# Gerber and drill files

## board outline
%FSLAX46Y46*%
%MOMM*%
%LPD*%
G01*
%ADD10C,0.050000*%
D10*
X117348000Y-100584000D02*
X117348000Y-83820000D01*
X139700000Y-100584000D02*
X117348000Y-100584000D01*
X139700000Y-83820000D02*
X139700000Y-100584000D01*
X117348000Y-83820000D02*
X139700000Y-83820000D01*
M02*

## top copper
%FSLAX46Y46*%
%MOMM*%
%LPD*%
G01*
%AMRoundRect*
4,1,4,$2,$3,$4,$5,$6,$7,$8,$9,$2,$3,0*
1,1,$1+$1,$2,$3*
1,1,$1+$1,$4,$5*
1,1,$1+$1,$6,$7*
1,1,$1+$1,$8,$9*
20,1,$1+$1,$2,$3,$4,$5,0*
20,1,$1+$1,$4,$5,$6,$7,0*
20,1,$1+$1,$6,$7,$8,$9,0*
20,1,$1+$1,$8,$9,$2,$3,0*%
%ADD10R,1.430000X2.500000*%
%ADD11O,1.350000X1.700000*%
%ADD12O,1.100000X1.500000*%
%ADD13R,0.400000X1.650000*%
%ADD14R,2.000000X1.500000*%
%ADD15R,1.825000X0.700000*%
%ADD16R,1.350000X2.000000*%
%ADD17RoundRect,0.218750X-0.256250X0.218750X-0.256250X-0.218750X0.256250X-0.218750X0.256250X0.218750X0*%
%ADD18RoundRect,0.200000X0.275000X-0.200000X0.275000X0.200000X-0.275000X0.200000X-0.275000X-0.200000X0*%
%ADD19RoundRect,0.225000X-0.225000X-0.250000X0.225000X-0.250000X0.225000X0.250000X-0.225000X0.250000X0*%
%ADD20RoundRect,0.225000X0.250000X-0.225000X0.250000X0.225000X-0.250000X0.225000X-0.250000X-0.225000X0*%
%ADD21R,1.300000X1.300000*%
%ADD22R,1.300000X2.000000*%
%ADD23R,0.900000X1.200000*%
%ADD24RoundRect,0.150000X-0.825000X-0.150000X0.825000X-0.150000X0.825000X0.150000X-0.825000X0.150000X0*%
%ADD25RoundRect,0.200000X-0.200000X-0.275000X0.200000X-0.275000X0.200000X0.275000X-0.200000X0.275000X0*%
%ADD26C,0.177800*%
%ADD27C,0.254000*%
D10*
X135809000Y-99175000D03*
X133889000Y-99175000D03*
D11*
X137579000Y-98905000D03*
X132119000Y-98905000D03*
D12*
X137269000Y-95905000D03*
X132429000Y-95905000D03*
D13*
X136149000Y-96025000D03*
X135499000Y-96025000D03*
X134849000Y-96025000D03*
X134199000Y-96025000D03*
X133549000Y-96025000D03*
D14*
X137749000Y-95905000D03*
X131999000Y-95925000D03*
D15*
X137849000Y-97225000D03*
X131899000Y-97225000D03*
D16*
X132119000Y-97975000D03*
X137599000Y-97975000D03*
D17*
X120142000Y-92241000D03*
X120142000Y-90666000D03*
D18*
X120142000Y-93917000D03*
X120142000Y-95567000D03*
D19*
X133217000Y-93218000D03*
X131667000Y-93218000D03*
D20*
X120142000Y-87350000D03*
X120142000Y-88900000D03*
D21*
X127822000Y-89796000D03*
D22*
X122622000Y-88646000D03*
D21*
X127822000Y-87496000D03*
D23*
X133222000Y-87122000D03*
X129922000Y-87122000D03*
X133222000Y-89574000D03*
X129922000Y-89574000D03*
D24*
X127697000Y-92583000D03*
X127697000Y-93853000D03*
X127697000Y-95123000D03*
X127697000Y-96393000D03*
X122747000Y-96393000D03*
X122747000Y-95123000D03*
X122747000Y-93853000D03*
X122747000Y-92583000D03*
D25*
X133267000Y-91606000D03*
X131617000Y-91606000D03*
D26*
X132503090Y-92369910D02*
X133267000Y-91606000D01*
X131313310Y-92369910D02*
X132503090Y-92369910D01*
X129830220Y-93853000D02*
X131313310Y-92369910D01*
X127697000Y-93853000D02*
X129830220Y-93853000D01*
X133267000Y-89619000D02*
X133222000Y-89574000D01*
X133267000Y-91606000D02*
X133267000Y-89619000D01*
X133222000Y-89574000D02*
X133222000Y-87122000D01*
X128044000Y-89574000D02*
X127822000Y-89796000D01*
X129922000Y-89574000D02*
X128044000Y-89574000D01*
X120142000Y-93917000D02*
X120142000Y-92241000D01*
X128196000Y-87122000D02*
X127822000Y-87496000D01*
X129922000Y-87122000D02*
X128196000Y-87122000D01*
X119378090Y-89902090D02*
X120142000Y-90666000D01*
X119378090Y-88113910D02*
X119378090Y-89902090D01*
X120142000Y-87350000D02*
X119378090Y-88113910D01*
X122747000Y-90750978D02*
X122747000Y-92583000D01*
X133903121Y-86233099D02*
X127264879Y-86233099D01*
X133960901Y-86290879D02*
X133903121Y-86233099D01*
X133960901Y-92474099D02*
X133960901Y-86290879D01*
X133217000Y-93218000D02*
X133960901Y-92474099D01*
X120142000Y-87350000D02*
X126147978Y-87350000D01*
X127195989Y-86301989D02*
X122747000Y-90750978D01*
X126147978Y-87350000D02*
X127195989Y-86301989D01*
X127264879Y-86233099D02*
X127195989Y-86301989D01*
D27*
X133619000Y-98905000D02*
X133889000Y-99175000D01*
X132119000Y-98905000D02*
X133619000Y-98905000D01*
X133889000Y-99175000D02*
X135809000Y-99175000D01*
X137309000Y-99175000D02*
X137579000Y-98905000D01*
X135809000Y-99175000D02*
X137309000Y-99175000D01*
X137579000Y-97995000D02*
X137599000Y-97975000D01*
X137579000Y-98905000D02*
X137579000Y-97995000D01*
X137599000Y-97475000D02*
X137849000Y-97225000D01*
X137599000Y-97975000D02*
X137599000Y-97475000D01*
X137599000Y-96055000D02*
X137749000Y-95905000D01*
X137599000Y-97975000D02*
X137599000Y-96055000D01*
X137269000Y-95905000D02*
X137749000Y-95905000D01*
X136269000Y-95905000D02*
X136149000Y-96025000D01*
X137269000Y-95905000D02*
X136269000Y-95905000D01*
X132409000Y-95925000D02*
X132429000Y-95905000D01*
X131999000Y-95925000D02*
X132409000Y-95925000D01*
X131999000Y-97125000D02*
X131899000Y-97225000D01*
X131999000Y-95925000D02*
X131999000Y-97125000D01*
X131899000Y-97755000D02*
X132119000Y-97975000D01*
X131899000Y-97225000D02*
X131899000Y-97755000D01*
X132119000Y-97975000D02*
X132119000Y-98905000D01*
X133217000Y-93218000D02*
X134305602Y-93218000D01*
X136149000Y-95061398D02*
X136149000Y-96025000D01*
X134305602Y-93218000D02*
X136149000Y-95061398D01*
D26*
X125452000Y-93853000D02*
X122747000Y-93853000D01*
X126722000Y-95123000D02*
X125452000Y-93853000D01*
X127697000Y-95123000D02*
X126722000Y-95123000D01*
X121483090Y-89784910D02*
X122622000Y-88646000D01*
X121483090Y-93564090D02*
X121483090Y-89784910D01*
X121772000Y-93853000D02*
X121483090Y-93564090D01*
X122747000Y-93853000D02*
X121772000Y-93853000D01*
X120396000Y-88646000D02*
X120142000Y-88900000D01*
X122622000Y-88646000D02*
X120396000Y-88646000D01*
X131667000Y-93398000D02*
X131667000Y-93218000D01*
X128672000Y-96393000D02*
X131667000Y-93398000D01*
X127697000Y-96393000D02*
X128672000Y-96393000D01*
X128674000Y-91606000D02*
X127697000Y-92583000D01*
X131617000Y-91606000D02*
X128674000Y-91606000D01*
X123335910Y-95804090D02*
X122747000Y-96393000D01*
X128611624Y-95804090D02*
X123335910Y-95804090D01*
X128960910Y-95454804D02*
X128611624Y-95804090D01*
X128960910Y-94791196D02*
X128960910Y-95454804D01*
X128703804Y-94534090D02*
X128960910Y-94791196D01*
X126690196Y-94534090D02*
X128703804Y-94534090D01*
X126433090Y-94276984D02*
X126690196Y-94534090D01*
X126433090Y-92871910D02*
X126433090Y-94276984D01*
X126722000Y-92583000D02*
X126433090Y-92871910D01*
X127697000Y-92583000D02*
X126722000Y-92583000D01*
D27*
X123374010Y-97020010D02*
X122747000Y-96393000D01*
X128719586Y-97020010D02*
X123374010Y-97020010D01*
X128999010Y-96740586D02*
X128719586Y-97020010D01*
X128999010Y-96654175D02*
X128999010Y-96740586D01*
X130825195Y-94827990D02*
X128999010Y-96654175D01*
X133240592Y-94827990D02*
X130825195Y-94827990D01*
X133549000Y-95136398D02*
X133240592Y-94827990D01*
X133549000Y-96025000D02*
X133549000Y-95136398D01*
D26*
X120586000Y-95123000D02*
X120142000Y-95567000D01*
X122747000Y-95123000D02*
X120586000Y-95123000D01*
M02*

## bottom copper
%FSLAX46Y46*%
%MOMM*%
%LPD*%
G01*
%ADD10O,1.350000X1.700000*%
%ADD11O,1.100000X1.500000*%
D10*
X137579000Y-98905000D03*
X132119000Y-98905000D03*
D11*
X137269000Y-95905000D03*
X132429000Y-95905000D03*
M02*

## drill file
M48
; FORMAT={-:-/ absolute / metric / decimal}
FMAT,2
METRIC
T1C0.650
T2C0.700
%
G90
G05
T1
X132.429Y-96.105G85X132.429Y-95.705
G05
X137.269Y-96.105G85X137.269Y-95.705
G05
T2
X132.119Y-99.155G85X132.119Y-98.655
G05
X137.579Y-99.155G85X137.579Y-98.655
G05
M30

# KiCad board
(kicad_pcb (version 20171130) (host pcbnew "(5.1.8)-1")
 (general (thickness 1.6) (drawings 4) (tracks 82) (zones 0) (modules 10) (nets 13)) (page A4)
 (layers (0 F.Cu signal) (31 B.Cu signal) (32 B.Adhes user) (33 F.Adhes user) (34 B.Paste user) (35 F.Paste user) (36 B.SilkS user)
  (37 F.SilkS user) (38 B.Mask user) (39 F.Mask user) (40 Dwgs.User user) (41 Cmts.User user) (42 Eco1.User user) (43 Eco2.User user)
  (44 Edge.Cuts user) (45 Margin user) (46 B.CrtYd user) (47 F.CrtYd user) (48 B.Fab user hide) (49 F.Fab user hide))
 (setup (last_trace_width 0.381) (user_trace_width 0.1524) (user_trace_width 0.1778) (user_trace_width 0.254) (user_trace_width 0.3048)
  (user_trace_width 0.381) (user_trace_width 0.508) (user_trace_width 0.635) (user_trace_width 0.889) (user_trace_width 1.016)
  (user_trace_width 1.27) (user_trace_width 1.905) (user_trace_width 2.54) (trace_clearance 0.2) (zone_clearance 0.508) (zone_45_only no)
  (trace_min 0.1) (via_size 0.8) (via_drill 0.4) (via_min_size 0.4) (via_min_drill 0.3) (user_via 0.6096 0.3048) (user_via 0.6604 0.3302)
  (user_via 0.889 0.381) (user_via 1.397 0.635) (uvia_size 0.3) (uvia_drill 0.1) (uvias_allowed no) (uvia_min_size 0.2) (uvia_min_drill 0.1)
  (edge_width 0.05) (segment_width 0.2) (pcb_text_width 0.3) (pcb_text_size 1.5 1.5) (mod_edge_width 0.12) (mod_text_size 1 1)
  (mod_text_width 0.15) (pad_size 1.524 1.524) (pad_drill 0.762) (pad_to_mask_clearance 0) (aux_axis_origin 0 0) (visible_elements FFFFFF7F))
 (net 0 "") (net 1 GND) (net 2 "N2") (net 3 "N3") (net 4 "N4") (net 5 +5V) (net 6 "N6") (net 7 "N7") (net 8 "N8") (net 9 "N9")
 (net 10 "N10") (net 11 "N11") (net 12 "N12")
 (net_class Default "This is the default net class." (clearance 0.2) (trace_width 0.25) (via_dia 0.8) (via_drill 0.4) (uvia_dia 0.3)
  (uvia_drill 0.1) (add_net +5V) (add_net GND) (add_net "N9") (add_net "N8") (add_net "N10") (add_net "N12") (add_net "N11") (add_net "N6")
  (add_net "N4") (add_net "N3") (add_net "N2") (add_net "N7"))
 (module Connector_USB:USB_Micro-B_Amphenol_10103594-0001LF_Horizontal (layer F.Cu) (at 134.874 97.79)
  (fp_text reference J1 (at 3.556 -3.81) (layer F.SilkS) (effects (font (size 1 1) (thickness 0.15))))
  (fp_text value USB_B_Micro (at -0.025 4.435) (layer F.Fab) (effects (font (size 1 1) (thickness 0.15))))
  (pad 6 smd rect (at 0.935 1.385 90) (size 2.5 1.43) (layers F.Cu F.Paste F.Mask) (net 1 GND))
  (pad 6 smd rect (at -0.985 1.385 90) (size 2.5 1.43) (layers F.Cu F.Paste F.Mask) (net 1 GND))
  (pad 6 thru_hole oval (at 2.705 1.115 90) (size 1.7 1.35) (drill oval 1.2 0.7) (layers *.Cu *.Mask) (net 1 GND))
  (pad 6 thru_hole oval (at -2.755 1.115 90) (size 1.7 1.35) (drill oval 1.2 0.7) (layers *.Cu *.Mask) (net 1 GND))
  (pad 6 thru_hole oval (at 2.395 -1.885 90) (size 1.5 1.1) (drill oval 1.05 0.65) (layers *.Cu *.Mask) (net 1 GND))
  (pad 6 thru_hole oval (at -2.445 -1.885 90) (size 1.5 1.1) (drill oval 1.05 0.65) (layers *.Cu *.Mask) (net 1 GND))
  (pad 5 smd rect (at 1.275 -1.765 90) (size 1.65 0.4) (layers F.Cu F.Paste F.Mask) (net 1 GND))
  (pad 4 smd rect (at 0.625 -1.765 90) (size 1.65 0.4) (layers F.Cu F.Paste F.Mask) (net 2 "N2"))
  (pad 3 smd rect (at -0.025 -1.765 90) (size 1.65 0.4) (layers F.Cu F.Paste F.Mask) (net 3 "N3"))
  (pad 2 smd rect (at -0.675 -1.765 90) (size 1.65 0.4) (layers F.Cu F.Paste F.Mask) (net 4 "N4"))
  (pad 1 smd rect (at -1.325 -1.765 90) (size 1.65 0.4) (layers F.Cu F.Paste F.Mask) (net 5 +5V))
  (pad 6 smd rect (at 2.875 -1.885) (size 2 1.5) (layers F.Cu F.Paste F.Mask) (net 1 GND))
  (pad 6 smd rect (at -2.875 -1.865) (size 2 1.5) (layers F.Cu F.Paste F.Mask) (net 1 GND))
  (pad 6 smd rect (at 2.975 -0.565) (size 1.825 0.7) (layers F.Cu F.Paste F.Mask) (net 1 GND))
  (pad 6 smd rect (at -2.975 -0.565) (size 1.825 0.7) (layers F.Cu F.Paste F.Mask) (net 1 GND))
  (pad 6 smd rect (at -2.755 0.185) (size 1.35 2) (layers F.Cu F.Paste F.Mask) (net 1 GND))
  (pad 6 smd rect (at 2.725 0.185) (size 1.35 2) (layers F.Cu F.Paste F.Mask) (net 1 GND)))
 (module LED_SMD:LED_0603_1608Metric (layer F.Cu) (at 120.142 91.4535 270)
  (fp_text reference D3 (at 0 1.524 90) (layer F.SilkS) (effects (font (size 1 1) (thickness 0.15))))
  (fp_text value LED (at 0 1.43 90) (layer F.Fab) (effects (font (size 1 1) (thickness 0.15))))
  (pad 2 smd roundrect (at 0.7875 0 270) (size 0.875 0.95) (layers F.Cu F.Paste F.Mask) (roundrect_rratio 0.25) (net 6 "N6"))
  (pad 1 smd roundrect (at -0.7875 0 270) (size 0.875 0.95) (layers F.Cu F.Paste F.Mask) (roundrect_rratio 0.25) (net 1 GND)))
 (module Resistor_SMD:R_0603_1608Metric (layer F.Cu) (at 120.142 94.742 90)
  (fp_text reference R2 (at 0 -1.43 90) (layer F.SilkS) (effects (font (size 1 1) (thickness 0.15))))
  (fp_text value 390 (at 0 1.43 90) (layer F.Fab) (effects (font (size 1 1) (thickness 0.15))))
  (pad 2 smd roundrect (at 0.825 0 90) (size 0.8 0.95) (layers F.Cu F.Paste F.Mask) (roundrect_rratio 0.25) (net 6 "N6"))
  (pad 1 smd roundrect (at -0.825 0 90) (size 0.8 0.95) (layers F.Cu F.Paste F.Mask) (roundrect_rratio 0.25) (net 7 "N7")))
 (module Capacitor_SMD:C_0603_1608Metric (layer F.Cu) (at 132.442 93.218)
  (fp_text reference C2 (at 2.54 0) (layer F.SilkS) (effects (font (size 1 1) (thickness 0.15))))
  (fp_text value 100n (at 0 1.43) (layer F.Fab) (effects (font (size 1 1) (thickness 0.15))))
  (pad 2 smd roundrect (at 0.775 0) (size 0.9 0.95) (layers F.Cu F.Paste F.Mask) (roundrect_rratio 0.25) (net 1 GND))
  (pad 1 smd roundrect (at -0.775 0) (size 0.9 0.95) (layers F.Cu F.Paste F.Mask) (roundrect_rratio 0.25) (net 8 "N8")))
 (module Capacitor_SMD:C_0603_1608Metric (layer F.Cu) (at 120.142 88.125 90)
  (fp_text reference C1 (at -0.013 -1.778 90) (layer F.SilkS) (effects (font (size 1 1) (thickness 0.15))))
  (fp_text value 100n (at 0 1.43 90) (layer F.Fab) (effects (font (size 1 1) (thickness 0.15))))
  (pad 2 smd roundrect (at 0.775 0 90) (size 0.9 0.95) (layers F.Cu F.Paste F.Mask) (roundrect_rratio 0.25) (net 1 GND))
  (pad 1 smd roundrect (at -0.775 0 90) (size 0.9 0.95) (layers F.Cu F.Paste F.Mask) (roundrect_rratio 0.25) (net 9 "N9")))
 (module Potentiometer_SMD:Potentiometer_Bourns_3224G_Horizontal (layer F.Cu) (at 125.222 88.646)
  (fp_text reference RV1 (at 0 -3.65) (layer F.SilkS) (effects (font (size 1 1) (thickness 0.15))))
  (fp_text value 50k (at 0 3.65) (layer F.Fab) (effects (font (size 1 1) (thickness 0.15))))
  (pad 3 smd rect (at 2.6 1.15) (size 1.3 1.3) (layers F.Cu F.Paste F.Mask) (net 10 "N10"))
  (pad 2 smd rect (at -2.6 0) (size 1.3 2) (layers F.Cu F.Paste F.Mask) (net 9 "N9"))
  (pad 1 smd rect (at 2.6 -1.15) (size 1.3 1.3) (layers F.Cu F.Paste F.Mask) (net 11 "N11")))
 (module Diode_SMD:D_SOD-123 (layer F.Cu) (at 131.572 87.122)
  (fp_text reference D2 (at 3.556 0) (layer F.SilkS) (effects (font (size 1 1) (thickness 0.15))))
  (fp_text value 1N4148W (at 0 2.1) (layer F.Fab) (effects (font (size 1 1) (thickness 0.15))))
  (pad 2 smd rect (at 1.65 0) (size 0.9 1.2) (layers F.Cu F.Paste F.Mask) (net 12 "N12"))
  (pad 1 smd rect (at -1.65 0) (size 0.9 1.2) (layers F.Cu F.Paste F.Mask) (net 11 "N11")))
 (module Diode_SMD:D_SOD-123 (layer F.Cu) (at 131.572 89.574)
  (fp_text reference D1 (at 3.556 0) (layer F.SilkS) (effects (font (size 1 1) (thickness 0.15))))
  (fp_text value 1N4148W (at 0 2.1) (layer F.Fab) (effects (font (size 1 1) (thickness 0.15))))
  (pad 2 smd rect (at 1.65 0) (size 0.9 1.2) (layers F.Cu F.Paste F.Mask) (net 12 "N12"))
  (pad 1 smd rect (at -1.65 0) (size 0.9 1.2) (layers F.Cu F.Paste F.Mask) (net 10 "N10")))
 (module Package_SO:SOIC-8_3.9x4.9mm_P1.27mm (layer F.Cu) (at 125.222 94.488)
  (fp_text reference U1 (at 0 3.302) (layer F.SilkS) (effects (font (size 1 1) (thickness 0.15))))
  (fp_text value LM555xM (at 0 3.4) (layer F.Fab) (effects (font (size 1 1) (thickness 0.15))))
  (pad 8 smd roundrect (at 2.475 -1.905) (size 1.95 0.6) (layers F.Cu F.Paste F.Mask) (roundrect_rratio 0.25) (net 5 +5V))
  (pad 7 smd roundrect (at 2.475 -0.635) (size 1.95 0.6) (layers F.Cu F.Paste F.Mask) (roundrect_rratio 0.25) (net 12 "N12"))
  (pad 6 smd roundrect (at 2.475 0.635) (size 1.95 0.6) (layers F.Cu F.Paste F.Mask) (roundrect_rratio 0.25) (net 9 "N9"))
  (pad 5 smd roundrect (at 2.475 1.905) (size 1.95 0.6) (layers F.Cu F.Paste F.Mask) (roundrect_rratio 0.25) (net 8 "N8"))
  (pad 4 smd roundrect (at -2.475 1.905) (size 1.95 0.6) (layers F.Cu F.Paste F.Mask) (roundrect_rratio 0.25) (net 5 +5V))
  (pad 3 smd roundrect (at -2.475 0.635) (size 1.95 0.6) (layers F.Cu F.Paste F.Mask) (roundrect_rratio 0.25) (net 7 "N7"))
  (pad 2 smd roundrect (at -2.475 -0.635) (size 1.95 0.6) (layers F.Cu F.Paste F.Mask) (roundrect_rratio 0.25) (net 9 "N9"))
  (pad 1 smd roundrect (at -2.475 -1.905) (size 1.95 0.6) (layers F.Cu F.Paste F.Mask) (roundrect_rratio 0.25) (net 1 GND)))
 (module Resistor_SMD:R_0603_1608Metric (layer F.Cu) (at 132.442 91.606)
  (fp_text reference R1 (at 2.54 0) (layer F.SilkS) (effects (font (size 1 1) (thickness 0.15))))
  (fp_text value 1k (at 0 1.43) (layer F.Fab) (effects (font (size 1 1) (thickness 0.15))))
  (pad 2 smd roundrect (at 0.825 0) (size 0.8 0.95) (layers F.Cu F.Paste F.Mask) (roundrect_rratio 0.25) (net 12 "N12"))
  (pad 1 smd roundrect (at -0.825 0) (size 0.8 0.95) (layers F.Cu F.Paste F.Mask) (roundrect_rratio 0.25) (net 5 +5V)))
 (gr_line (start 117.348 100.584) (end 117.348 83.82) (layer Edge.Cuts) (width 0.05))
 (gr_line (start 139.7 100.584) (end 117.348 100.584) (layer Edge.Cuts) (width 0.05))
 (gr_line (start 139.7 83.82) (end 139.7 100.584) (layer Edge.Cuts) (width 0.05))
 (gr_line (start 117.348 83.82) (end 139.7 83.82) (layer Edge.Cuts) (width 0.05))
 (segment (start 132.50309 92.36991) (end 133.267 91.606) (width 0.1778) (layer F.Cu) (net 12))
 (segment (start 131.31331 92.36991) (end 132.50309 92.36991) (width 0.1778) (layer F.Cu) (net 12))
 (segment (start 129.83022 93.853) (end 131.31331 92.36991) (width 0.1778) (layer F.Cu) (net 12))
 (segment (start 127.697 93.853) (end 129.83022 93.853) (width 0.1778) (layer F.Cu) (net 12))
 (segment (start 133.267 89.619) (end 133.222 89.574) (width 0.1778) (layer F.Cu) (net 12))
 (segment (start 133.267 91.606) (end 133.267 89.619) (width 0.1778) (layer F.Cu) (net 12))
 (segment (start 133.222 89.574) (end 133.222 87.122) (width 0.1778) (layer F.Cu) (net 12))
 (segment (start 128.044 89.574) (end 127.822 89.796) (width 0.1778) (layer F.Cu) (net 10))
 (segment (start 129.922 89.574) (end 128.044 89.574) (width 0.1778) (layer F.Cu) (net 10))
 (segment (start 120.142 93.917) (end 120.142 92.241) (width 0.1778) (layer F.Cu) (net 6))
 (segment (start 128.196 87.122) (end 127.822 87.496) (width 0.1778) (layer F.Cu) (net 11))
 (segment (start 129.922 87.122) (end 128.196 87.122) (width 0.1778) (layer F.Cu) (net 11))
 (segment (start 119.37809 89.90209) (end 120.142 90.666) (width 0.1778) (layer F.Cu) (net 1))
 (segment (start 119.37809 88.11391) (end 119.37809 89.90209) (width 0.1778) (layer F.Cu) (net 1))
 (segment (start 120.142 87.35) (end 119.37809 88.11391) (width 0.1778) (layer F.Cu) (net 1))
 (segment (start 122.747 90.750978) (end 122.747 92.583) (width 0.1778) (layer F.Cu) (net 1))
 (segment (start 133.903121 86.233099) (end 127.264879 86.233099) (width 0.1778) (layer F.Cu) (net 1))
 (segment (start 133.960901 86.290879) (end 133.903121 86.233099) (width 0.1778) (layer F.Cu) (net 1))
 (segment (start 133.960901 92.474099) (end 133.960901 86.290879) (width 0.1778) (layer F.Cu) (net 1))
 (segment (start 133.217 93.218) (end 133.960901 92.474099) (width 0.1778) (layer F.Cu) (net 1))
 (segment (start 120.142 87.35) (end 126.147978 87.35) (width 0.1778) (layer F.Cu) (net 1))
 (segment (start 127.195989 86.301989) (end 122.747 90.750978) (width 0.1778) (layer F.Cu) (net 1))
 (segment (start 126.147978 87.35) (end 127.195989 86.301989) (width 0.1778) (layer F.Cu) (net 1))
 (segment (start 127.264879 86.233099) (end 127.195989 86.301989) (width 0.1778) (layer F.Cu) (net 1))
 (segment (start 133.619 98.905) (end 133.889 99.175) (width 0.254) (layer F.Cu) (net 1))
 (segment (start 132.119 98.905) (end 133.619 98.905) (width 0.254) (layer F.Cu) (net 1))
 (segment (start 133.889 99.175) (end 135.809 99.175) (width 0.254) (layer F.Cu) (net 1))
 (segment (start 137.309 99.175) (end 137.579 98.905) (width 0.254) (layer F.Cu) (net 1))
 (segment (start 135.809 99.175) (end 137.309 99.175) (width 0.254) (layer F.Cu) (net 1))
 (segment (start 137.579 97.995) (end 137.599 97.975) (width 0.254) (layer F.Cu) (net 1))
 (segment (start 137.579 98.905) (end 137.579 97.995) (width 0.254) (layer F.Cu) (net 1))
 (segment (start 137.599 97.475) (end 137.849 97.225) (width 0.254) (layer F.Cu) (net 1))
 (segment (start 137.599 97.975) (end 137.599 97.475) (width 0.254) (layer F.Cu) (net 1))
 (segment (start 137.599 96.055) (end 137.749 95.905) (width 0.254) (layer F.Cu) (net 1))
 (segment (start 137.599 97.975) (end 137.599 96.055) (width 0.254) (layer F.Cu) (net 1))
 (segment (start 137.269 95.905) (end 137.749 95.905) (width 0.254) (layer F.Cu) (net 1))
 (segment (start 136.269 95.905) (end 136.149 96.025) (width 0.254) (layer F.Cu) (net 1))
 (segment (start 137.269 95.905) (end 136.269 95.905) (width 0.254) (layer F.Cu) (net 1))
 (segment (start 132.409 95.925) (end 132.429 95.905) (width 0.254) (layer F.Cu) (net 1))
 (segment (start 131.999 95.925) (end 132.409 95.925) (width 0.254) (layer F.Cu) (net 1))
 (segment (start 131.999 97.125) (end 131.899 97.225) (width 0.254) (layer F.Cu) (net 1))
 (segment (start 131.999 95.925) (end 131.999 97.125) (width 0.254) (layer F.Cu) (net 1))
 (segment (start 131.899 97.755) (end 132.119 97.975) (width 0.254) (layer F.Cu) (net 1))
 (segment (start 131.899 97.225) (end 131.899 97.755) (width 0.254) (layer F.Cu) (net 1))
 (segment (start 132.119 97.975) (end 132.119 98.905) (width 0.254) (layer F.Cu) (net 1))
 (segment (start 133.217 93.218) (end 134.305602 93.218) (width 0.254) (layer F.Cu) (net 1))
 (segment (start 136.149 95.061398) (end 136.149 96.025) (width 0.254) (layer F.Cu) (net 1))
 (segment (start 134.305602 93.218) (end 136.149 95.061398) (width 0.254) (layer F.Cu) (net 1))
 (segment (start 125.452 93.853) (end 122.747 93.853) (width 0.1778) (layer F.Cu) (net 9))
 (segment (start 126.722 95.123) (end 125.452 93.853) (width 0.1778) (layer F.Cu) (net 9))
 (segment (start 127.697 95.123) (end 126.722 95.123) (width 0.1778) (layer F.Cu) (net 9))
 (segment (start 121.48309 89.78491) (end 122.622 88.646) (width 0.1778) (layer F.Cu) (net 9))
 (segment (start 121.48309 93.56409) (end 121.48309 89.78491) (width 0.1778) (layer F.Cu) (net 9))
 (segment (start 121.772 93.853) (end 121.48309 93.56409) (width 0.1778) (layer F.Cu) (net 9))
 (segment (start 122.747 93.853) (end 121.772 93.853) (width 0.1778) (layer F.Cu) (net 9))
 (segment (start 120.396 88.646) (end 120.142 88.9) (width 0.1778) (layer F.Cu) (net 9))
 (segment (start 122.622 88.646) (end 120.396 88.646) (width 0.1778) (layer F.Cu) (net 9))
 (segment (start 131.667 93.398) (end 131.667 93.218) (width 0.1778) (layer F.Cu) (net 8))
 (segment (start 128.672 96.393) (end 131.667 93.398) (width 0.1778) (layer F.Cu) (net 8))
 (segment (start 127.697 96.393) (end 128.672 96.393) (width 0.1778) (layer F.Cu) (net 8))
 (segment (start 128.674 91.606) (end 127.697 92.583) (width 0.1778) (layer F.Cu) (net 5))
 (segment (start 131.617 91.606) (end 128.674 91.606) (width 0.1778) (layer F.Cu) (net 5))
 (segment (start 123.33591 95.80409) (end 122.747 96.393) (width 0.1778) (layer F.Cu) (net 5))
 (segment (start 128.611624 95.80409) (end 123.33591 95.80409) (width 0.1778) (layer F.Cu) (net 5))
 (segment (start 128.96091 95.454804) (end 128.611624 95.80409) (width 0.1778) (layer F.Cu) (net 5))
 (segment (start 128.96091 94.791196) (end 128.96091 95.454804) (width 0.1778) (layer F.Cu) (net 5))
 (segment (start 128.703804 94.53409) (end 128.96091 94.791196) (width 0.1778) (layer F.Cu) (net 5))
 (segment (start 126.690196 94.53409) (end 128.703804 94.53409) (width 0.1778) (layer F.Cu) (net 5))
 (segment (start 126.43309 94.276984) (end 126.690196 94.53409) (width 0.1778) (layer F.Cu) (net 5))
 (segment (start 126.43309 92.87191) (end 126.43309 94.276984) (width 0.1778) (layer F.Cu) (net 5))
 (segment (start 126.722 92.583) (end 126.43309 92.87191) (width 0.1778) (layer F.Cu) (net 5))
 (segment (start 127.697 92.583) (end 126.722 92.583) (width 0.1778) (layer F.Cu) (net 5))
 (segment (start 123.37401 97.02001) (end 122.747 96.393) (width 0.254) (layer F.Cu) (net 5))
 (segment (start 128.719586 97.02001) (end 123.37401 97.02001) (width 0.254) (layer F.Cu) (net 5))
 (segment (start 128.99901 96.740586) (end 128.719586 97.02001) (width 0.254) (layer F.Cu) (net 5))
 (segment (start 128.99901 96.654175) (end 128.99901 96.740586) (width 0.254) (layer F.Cu) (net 5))
 (segment (start 130.825195 94.82799) (end 128.99901 96.654175) (width 0.254) (layer F.Cu) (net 5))
 (segment (start 133.240592 94.82799) (end 130.825195 94.82799) (width 0.254) (layer F.Cu) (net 5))
 (segment (start 133.549 95.136398) (end 133.240592 94.82799) (width 0.254) (layer F.Cu) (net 5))
 (segment (start 133.549 96.025) (end 133.549 95.136398) (width 0.254) (layer F.Cu) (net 5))
 (segment (start 120.586 95.123) (end 120.142 95.567) (width 0.1778) (layer F.Cu) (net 7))
 (segment (start 122.747 95.123) (end 120.586 95.123) (width 0.1778) (layer F.Cu) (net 7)))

